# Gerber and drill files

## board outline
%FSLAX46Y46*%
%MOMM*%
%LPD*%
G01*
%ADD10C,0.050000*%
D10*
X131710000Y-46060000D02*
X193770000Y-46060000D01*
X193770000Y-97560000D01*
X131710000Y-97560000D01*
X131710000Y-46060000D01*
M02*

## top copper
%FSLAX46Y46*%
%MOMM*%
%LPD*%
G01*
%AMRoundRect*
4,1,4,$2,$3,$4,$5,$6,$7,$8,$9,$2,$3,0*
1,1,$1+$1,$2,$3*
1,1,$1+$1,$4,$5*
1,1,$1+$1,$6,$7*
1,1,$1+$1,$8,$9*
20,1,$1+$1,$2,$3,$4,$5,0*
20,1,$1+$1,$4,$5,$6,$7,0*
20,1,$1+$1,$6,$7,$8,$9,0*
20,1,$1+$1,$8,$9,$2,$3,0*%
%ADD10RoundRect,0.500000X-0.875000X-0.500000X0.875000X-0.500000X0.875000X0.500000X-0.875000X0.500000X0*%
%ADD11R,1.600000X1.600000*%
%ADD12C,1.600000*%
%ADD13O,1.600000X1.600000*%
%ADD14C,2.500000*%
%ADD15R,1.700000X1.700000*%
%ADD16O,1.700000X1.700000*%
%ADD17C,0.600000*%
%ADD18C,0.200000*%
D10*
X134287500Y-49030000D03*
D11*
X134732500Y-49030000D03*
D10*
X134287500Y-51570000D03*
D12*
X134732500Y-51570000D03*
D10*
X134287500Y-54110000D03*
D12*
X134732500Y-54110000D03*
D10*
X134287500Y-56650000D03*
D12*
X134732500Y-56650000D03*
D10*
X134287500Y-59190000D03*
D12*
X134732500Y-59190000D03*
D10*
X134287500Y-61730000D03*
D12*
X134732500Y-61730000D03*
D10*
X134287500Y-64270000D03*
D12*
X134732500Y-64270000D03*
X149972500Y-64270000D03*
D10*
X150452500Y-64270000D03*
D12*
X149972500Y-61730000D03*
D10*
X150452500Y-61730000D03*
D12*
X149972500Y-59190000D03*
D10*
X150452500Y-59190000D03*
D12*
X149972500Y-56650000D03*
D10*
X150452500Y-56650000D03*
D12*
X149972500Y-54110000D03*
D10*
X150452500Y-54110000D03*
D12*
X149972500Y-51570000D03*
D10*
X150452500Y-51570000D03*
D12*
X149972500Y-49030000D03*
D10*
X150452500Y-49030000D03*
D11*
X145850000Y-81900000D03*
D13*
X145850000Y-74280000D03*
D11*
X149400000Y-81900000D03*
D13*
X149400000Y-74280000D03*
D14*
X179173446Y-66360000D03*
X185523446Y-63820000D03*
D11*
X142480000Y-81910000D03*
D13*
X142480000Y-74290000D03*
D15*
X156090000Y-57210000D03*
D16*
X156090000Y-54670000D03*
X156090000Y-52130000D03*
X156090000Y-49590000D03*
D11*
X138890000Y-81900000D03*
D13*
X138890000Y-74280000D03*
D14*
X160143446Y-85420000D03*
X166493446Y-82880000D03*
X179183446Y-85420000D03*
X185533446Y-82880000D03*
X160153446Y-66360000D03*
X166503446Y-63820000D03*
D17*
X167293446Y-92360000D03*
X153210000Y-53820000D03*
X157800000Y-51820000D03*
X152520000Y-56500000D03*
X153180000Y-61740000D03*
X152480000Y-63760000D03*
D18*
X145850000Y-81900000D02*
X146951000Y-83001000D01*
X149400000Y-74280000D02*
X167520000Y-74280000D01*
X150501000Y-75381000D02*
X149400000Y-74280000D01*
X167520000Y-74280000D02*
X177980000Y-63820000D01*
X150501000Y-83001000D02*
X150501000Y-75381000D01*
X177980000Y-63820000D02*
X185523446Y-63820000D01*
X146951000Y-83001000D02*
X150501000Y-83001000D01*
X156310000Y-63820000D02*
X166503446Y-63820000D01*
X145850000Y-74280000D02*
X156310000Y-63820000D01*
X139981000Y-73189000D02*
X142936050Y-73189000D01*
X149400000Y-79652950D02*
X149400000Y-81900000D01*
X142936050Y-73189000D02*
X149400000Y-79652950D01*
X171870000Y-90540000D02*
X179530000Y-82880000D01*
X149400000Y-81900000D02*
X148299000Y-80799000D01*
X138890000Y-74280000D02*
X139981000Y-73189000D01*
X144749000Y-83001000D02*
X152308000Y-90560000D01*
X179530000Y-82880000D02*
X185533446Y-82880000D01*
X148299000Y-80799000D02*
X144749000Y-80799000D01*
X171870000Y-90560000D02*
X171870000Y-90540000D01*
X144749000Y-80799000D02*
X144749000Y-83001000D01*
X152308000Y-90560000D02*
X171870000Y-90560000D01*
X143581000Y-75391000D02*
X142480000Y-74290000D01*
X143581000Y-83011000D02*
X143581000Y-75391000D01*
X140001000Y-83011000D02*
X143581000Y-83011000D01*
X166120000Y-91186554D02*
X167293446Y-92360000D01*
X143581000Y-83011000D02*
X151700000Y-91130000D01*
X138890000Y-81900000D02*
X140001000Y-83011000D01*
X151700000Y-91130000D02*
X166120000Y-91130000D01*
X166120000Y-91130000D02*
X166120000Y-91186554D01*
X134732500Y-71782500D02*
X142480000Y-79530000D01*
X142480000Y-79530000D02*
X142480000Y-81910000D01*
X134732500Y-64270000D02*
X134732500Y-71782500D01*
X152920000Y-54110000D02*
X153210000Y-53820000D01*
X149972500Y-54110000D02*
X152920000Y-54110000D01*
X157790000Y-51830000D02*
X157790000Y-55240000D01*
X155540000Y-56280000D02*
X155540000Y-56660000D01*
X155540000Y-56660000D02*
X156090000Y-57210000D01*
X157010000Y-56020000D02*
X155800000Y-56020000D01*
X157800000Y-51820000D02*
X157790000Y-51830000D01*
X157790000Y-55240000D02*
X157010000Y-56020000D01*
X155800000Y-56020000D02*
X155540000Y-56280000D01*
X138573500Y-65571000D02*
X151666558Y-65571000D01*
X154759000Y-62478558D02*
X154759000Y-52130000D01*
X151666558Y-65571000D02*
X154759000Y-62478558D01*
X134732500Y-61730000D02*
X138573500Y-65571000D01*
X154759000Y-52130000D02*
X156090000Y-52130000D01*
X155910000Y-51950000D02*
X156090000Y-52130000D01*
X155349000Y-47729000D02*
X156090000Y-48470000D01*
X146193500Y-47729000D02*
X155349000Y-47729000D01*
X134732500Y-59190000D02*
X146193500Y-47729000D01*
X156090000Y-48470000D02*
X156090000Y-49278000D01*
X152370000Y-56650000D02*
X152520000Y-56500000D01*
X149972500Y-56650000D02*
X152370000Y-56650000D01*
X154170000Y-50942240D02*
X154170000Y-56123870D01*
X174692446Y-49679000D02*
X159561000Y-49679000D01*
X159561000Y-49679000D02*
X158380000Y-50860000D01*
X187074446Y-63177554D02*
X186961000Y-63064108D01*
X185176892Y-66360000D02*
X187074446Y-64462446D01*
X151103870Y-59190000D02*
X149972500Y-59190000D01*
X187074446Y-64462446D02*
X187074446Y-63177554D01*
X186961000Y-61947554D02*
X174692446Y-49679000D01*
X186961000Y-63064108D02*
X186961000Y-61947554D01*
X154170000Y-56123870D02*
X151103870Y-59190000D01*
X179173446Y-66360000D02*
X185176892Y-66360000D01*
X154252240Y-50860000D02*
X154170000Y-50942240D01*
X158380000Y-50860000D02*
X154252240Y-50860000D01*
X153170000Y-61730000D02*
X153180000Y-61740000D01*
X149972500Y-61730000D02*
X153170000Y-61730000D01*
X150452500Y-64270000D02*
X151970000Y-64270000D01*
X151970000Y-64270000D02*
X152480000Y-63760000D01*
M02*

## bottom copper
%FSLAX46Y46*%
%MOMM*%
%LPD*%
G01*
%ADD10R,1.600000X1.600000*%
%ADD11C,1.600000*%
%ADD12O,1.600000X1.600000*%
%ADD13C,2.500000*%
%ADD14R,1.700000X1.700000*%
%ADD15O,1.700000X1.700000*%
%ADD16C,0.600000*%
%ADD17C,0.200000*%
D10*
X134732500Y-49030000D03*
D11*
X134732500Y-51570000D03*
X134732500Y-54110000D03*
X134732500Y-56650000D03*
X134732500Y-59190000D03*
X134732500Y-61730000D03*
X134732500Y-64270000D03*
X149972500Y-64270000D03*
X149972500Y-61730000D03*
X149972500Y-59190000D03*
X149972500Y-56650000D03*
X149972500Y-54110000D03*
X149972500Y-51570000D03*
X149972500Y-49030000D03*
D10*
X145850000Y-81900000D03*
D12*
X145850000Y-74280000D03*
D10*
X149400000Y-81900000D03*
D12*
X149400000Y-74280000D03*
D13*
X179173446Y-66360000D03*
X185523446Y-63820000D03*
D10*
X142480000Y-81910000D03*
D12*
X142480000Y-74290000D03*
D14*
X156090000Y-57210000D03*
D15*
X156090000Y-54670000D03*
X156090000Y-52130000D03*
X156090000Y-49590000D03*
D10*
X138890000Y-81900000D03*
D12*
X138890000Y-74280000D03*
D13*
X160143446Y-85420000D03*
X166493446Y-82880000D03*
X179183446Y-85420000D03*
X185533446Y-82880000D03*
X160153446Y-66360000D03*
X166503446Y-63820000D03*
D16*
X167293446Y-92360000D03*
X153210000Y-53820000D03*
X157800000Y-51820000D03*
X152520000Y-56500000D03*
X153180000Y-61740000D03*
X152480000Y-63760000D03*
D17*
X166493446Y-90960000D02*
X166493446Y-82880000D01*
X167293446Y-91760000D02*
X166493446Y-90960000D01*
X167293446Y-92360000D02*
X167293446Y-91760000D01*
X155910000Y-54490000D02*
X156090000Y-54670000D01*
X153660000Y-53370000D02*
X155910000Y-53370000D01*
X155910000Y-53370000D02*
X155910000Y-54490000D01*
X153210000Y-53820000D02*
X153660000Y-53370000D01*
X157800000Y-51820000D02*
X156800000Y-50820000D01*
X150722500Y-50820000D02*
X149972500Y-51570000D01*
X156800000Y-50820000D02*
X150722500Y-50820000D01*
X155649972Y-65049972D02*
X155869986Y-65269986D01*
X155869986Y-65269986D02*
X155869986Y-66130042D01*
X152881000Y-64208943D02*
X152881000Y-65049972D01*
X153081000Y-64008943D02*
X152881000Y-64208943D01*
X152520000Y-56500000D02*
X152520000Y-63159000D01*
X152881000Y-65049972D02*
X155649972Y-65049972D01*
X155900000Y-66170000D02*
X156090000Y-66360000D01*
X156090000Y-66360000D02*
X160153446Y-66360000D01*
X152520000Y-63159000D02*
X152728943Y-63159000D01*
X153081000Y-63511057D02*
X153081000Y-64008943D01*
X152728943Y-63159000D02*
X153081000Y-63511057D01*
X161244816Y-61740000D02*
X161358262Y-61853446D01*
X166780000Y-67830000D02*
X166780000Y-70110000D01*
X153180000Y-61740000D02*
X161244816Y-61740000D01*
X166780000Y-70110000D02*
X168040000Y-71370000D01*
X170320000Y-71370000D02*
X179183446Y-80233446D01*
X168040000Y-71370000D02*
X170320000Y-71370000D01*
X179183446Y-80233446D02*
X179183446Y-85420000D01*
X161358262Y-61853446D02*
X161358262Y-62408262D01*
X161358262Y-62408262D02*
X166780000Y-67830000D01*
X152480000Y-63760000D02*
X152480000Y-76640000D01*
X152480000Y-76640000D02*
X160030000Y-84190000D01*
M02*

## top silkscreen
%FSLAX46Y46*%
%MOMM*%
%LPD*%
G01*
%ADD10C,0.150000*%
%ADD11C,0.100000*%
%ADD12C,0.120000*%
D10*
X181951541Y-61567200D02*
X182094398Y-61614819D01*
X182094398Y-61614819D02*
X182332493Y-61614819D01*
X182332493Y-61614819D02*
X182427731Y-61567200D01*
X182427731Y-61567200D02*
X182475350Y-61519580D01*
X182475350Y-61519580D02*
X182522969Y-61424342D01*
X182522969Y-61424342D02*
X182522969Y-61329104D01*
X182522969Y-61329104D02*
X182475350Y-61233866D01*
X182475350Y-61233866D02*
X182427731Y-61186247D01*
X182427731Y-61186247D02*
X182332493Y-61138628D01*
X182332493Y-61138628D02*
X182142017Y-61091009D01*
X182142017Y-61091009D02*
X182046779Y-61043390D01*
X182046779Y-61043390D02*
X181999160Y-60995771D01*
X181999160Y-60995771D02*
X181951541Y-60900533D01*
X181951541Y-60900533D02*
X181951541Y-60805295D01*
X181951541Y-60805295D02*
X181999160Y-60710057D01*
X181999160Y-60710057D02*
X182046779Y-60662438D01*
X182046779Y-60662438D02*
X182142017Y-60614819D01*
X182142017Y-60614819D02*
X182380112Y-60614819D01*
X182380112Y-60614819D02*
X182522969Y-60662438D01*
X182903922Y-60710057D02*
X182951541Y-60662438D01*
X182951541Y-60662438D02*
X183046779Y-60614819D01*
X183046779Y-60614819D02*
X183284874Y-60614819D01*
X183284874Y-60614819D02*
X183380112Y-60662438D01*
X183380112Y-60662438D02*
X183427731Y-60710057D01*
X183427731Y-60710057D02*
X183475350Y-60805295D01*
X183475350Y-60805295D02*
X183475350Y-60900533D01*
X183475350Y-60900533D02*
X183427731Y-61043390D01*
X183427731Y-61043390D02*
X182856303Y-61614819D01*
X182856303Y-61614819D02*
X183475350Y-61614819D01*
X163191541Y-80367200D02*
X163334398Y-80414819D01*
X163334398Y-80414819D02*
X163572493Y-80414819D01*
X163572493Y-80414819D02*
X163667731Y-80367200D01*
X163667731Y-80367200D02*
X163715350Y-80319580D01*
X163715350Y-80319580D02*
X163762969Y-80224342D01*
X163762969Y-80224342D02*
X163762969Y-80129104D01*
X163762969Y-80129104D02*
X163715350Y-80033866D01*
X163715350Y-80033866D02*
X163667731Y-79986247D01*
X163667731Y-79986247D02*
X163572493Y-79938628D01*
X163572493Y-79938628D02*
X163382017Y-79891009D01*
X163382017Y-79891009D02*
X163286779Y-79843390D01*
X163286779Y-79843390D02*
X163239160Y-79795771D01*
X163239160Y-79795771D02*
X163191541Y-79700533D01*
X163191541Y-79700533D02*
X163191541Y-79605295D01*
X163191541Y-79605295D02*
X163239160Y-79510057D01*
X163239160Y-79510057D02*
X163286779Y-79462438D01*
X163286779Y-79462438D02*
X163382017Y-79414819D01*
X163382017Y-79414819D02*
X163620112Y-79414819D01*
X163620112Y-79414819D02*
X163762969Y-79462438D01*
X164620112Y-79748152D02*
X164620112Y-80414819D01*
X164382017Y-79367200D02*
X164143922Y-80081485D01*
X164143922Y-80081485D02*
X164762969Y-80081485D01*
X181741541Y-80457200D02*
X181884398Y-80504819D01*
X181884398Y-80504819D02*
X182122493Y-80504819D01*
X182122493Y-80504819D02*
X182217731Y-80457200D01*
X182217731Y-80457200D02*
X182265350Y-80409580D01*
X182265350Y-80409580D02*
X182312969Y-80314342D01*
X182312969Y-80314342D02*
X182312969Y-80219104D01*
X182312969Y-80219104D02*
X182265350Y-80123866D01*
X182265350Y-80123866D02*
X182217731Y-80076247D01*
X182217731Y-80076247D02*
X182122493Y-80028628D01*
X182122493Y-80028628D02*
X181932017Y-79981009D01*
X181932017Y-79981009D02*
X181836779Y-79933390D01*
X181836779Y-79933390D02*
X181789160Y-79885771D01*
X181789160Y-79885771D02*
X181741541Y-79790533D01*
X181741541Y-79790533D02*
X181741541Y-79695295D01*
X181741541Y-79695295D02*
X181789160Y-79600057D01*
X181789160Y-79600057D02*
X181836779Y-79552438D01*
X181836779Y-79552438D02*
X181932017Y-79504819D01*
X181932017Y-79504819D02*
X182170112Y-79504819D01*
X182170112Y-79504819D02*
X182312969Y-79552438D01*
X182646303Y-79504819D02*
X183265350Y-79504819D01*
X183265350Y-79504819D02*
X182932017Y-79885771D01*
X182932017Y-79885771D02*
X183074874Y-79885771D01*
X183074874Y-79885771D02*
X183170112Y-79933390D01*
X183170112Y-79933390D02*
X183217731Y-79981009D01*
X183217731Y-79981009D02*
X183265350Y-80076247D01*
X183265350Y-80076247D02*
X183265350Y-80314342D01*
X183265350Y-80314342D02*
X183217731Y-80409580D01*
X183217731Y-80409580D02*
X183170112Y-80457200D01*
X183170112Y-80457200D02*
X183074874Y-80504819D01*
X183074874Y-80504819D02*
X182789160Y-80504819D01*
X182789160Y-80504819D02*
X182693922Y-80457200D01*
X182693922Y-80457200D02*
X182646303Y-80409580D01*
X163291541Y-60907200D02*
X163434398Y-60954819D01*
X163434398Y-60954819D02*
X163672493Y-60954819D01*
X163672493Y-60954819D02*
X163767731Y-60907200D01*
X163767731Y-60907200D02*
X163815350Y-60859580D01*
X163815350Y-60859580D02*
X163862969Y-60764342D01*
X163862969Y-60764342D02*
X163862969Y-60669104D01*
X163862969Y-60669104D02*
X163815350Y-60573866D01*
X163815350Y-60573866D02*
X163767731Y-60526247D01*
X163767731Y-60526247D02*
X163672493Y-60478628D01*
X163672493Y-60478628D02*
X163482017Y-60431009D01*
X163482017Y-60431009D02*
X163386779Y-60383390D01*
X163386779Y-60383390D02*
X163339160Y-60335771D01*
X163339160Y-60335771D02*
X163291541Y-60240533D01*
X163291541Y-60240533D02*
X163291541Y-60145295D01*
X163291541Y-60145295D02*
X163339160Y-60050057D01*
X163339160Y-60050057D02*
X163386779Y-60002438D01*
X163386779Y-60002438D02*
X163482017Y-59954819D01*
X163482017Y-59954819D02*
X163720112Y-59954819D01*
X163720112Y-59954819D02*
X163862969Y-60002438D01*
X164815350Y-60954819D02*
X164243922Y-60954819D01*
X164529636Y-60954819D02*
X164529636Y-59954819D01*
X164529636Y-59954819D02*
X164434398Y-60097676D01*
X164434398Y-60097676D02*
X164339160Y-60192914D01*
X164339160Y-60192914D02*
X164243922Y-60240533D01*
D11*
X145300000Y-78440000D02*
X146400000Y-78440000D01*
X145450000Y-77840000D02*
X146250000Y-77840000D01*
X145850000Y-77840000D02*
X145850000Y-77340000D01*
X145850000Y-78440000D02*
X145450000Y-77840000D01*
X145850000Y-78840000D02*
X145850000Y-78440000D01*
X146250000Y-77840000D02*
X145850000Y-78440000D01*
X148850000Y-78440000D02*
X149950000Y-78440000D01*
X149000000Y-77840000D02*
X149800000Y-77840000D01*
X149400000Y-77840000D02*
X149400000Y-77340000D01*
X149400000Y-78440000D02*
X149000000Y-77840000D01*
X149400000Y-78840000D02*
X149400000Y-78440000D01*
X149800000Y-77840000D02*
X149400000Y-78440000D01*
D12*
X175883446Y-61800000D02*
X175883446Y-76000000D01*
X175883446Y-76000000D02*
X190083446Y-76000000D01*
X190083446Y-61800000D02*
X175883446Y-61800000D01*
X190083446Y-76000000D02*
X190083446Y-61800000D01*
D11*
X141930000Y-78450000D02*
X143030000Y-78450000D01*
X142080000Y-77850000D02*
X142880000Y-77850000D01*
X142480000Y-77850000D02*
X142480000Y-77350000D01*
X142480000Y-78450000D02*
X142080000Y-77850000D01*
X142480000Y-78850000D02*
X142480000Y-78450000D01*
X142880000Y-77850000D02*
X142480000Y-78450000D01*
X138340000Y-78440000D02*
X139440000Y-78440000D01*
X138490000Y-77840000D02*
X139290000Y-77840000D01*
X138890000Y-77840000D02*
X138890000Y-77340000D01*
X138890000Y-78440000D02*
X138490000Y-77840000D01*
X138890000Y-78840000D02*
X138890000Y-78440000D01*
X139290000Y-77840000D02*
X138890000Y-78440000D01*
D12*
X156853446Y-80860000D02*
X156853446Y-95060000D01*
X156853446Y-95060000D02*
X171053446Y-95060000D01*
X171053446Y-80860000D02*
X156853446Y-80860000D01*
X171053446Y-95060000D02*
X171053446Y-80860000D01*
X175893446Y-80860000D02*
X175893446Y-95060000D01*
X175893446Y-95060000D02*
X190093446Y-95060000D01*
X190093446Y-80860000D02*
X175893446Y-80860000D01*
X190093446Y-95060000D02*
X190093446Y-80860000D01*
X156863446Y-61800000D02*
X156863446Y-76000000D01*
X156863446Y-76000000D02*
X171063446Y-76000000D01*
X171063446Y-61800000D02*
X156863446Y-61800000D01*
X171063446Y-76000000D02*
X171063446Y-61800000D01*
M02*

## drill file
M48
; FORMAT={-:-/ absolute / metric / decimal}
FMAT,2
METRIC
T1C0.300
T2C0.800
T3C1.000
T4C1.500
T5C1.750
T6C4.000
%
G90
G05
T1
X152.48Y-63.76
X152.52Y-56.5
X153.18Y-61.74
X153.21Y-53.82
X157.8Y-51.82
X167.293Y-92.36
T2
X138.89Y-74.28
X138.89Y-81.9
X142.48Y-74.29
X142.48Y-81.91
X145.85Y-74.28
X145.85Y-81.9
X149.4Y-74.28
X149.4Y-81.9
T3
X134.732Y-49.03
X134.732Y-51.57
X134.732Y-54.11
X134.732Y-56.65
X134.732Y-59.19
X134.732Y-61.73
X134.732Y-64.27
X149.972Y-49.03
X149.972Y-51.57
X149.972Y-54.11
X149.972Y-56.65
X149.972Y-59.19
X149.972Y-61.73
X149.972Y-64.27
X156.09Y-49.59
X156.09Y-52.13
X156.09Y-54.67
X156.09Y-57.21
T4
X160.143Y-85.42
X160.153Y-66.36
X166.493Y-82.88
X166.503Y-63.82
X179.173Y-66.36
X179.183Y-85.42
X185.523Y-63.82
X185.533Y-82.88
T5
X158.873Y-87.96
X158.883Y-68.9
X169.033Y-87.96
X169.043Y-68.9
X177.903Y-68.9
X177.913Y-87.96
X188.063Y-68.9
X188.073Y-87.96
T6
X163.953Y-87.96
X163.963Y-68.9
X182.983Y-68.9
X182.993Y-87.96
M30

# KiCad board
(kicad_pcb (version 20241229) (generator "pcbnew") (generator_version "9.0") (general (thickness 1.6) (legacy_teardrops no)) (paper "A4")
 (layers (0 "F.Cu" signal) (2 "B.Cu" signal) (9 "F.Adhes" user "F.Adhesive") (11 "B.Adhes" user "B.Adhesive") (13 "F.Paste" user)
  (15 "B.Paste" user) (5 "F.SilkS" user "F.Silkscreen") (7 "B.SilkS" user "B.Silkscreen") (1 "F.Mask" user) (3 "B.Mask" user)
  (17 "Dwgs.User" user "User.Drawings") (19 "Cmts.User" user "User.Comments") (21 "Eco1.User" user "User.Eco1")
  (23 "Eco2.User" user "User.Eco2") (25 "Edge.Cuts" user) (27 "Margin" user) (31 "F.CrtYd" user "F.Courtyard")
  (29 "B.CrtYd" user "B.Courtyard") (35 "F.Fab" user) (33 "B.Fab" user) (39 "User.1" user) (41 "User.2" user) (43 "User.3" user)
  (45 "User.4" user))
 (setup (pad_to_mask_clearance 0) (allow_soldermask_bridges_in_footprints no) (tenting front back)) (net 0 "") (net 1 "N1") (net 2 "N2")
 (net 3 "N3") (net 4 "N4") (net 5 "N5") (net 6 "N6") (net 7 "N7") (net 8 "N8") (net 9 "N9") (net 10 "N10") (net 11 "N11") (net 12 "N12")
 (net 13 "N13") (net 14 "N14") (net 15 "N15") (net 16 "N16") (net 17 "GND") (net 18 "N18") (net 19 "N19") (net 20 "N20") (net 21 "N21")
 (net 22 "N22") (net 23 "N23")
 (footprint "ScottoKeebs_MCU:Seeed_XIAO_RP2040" (layer "F.Cu") (at 142.3525 56.65)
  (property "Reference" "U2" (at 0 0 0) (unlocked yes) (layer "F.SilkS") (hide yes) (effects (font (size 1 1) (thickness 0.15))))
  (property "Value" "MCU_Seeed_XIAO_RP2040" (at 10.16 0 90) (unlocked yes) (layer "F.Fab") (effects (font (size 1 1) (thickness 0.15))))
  (pad "1" smd roundrect (at -8.065 -7.62) (size 2.75 2) (layers "F.Cu" "F.Mask" "F.Paste") (roundrect_rratio 0.25) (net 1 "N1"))
  (pad "1" thru_hole rect (at -7.62 -7.62 90) (size 1.6 1.6) (drill 1) (layers "*.Cu" "*.Mask") (remove_unused_layers no) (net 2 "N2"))
  (pad "2" smd roundrect (at -8.065 -5.08) (size 2.75 2) (layers "F.Cu" "F.Mask" "F.Paste") (roundrect_rratio 0.25) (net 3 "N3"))
  (pad "2" thru_hole circle (at -7.62 -5.08 90) (size 1.6 1.6) (drill 1) (layers "*.Cu" "*.Mask") (remove_unused_layers no) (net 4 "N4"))
  (pad "3" smd roundrect (at -8.065 -2.54) (size 2.75 2) (layers "F.Cu" "F.Mask" "F.Paste") (roundrect_rratio 0.25) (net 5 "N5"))
  (pad "3" thru_hole circle (at -7.62 -2.54 90) (size 1.6 1.6) (drill 1) (layers "*.Cu" "*.Mask") (remove_unused_layers no) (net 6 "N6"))
  (pad "4" smd roundrect (at -8.065 0) (size 2.75 2) (layers "F.Cu" "F.Mask" "F.Paste") (roundrect_rratio 0.25) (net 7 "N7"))
  (pad "4" thru_hole circle (at -7.62 0 90) (size 1.6 1.6) (drill 1) (layers "*.Cu" "*.Mask") (remove_unused_layers no) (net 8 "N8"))
  (pad "5" smd roundrect (at -8.065 2.54) (size 2.75 2) (layers "F.Cu" "F.Mask" "F.Paste") (roundrect_rratio 0.25) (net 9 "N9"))
  (pad "5" thru_hole circle (at -7.62 2.54 90) (size 1.6 1.6) (drill 1) (layers "*.Cu" "*.Mask") (remove_unused_layers no) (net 9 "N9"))
  (pad "6" smd roundrect (at -8.065 5.08) (size 2.75 2) (layers "F.Cu" "F.Mask" "F.Paste") (roundrect_rratio 0.25) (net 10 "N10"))
  (pad "6" thru_hole circle (at -7.62 5.08 90) (size 1.6 1.6) (drill 1) (layers "*.Cu" "*.Mask") (remove_unused_layers no) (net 10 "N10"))
  (pad "7" smd roundrect (at -8.065 7.62) (size 2.75 2) (layers "F.Cu" "F.Mask" "F.Paste") (roundrect_rratio 0.25) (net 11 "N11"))
  (pad "7" thru_hole circle (at -7.62 7.62 90) (size 1.6 1.6) (drill 1) (layers "*.Cu" "*.Mask") (remove_unused_layers no) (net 11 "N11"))
  (pad "8" thru_hole circle (at 7.62 7.62 90) (size 1.6 1.6) (drill 1) (layers "*.Cu" "*.Mask") (remove_unused_layers no) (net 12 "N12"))
  (pad "8" smd roundrect (at 8.1 7.62) (size 2.75 2) (layers "F.Cu" "F.Mask" "F.Paste") (roundrect_rratio 0.25) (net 12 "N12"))
  (pad "9" thru_hole circle (at 7.62 5.08 90) (size 1.6 1.6) (drill 1) (layers "*.Cu" "*.Mask") (remove_unused_layers no) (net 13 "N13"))
  (pad "9" smd roundrect (at 8.1 5.08) (size 2.75 2) (layers "F.Cu" "F.Mask" "F.Paste") (roundrect_rratio 0.25) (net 13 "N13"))
  (pad "10" thru_hole circle (at 7.62 2.54 90) (size 1.6 1.6) (drill 1) (layers "*.Cu" "*.Mask") (remove_unused_layers no) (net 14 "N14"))
  (pad "10" smd roundrect (at 8.1 2.54) (size 2.75 2) (layers "F.Cu" "F.Mask" "F.Paste") (roundrect_rratio 0.25) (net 14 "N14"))
  (pad "11" thru_hole circle (at 7.62 0 90) (size 1.6 1.6) (drill 1) (layers "*.Cu" "*.Mask") (remove_unused_layers no) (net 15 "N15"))
  (pad "11" smd roundrect (at 8.1 0) (size 2.75 2) (layers "F.Cu" "F.Mask" "F.Paste") (roundrect_rratio 0.25) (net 15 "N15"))
  (pad "12" thru_hole circle (at 7.62 -2.54 90) (size 1.6 1.6) (drill 1) (layers "*.Cu" "*.Mask") (remove_unused_layers no) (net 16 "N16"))
  (pad "12" smd roundrect (at 8.1 -2.54) (size 2.75 2) (layers "F.Cu" "F.Mask" "F.Paste") (roundrect_rratio 0.25) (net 16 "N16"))
  (pad "13" thru_hole circle (at 7.62 -5.08 90) (size 1.6 1.6) (drill 1) (layers "*.Cu" "*.Mask") (remove_unused_layers no) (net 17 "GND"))
  (pad "13" smd roundrect (at 8.1 -5.08) (size 2.75 2) (layers "F.Cu" "F.Mask" "F.Paste") (roundrect_rratio 0.25) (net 17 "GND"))
  (pad "14" thru_hole circle (at 7.62 -7.62 90) (size 1.6 1.6) (drill 1) (layers "*.Cu" "*.Mask") (remove_unused_layers no) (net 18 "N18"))
  (pad "14" smd roundrect (at 8.1 -7.62) (size 2.75 2) (layers "F.Cu" "F.Mask" "F.Paste") (roundrect_rratio 0.25) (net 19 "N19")))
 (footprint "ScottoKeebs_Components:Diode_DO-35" (layer "F.Cu") (at 145.85 81.9 90)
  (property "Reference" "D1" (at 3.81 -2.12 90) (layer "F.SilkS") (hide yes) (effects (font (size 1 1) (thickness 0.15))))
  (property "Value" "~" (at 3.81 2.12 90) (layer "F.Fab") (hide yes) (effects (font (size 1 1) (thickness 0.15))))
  (fp_line (start 3.46 -0.55) (end 3.46 0.55) (stroke (width 0.1) (type solid)) (layer "F.SilkS"))
  (fp_line (start 4.06 -0.4) (end 4.06 0.4) (stroke (width 0.1) (type solid)) (layer "F.SilkS"))
  (fp_line (start 4.06 0) (end 4.56 0) (stroke (width 0.1) (type solid)) (layer "F.SilkS"))
  (fp_line (start 3.46 0) (end 4.06 -0.4) (stroke (width 0.1) (type solid)) (layer "F.SilkS"))
  (fp_line (start 3.06 0) (end 3.46 0) (stroke (width 0.1) (type solid)) (layer "F.SilkS"))
  (fp_line (start 4.06 0.4) (end 3.46 0) (stroke (width 0.1) (type solid)) (layer "F.SilkS"))
  (pad "1" thru_hole rect (at 0 0 90) (size 1.6 1.6) (drill 0.8) (layers "*.Cu" "*.Mask") (remove_unused_layers no) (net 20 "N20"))
  (pad "2" thru_hole oval (at 7.62 0 90) (size 1.6 1.6) (drill 0.8) (layers "*.Cu" "*.Mask") (remove_unused_layers no) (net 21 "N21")))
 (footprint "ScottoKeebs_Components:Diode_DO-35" (layer "F.Cu") (at 149.4 81.9 90)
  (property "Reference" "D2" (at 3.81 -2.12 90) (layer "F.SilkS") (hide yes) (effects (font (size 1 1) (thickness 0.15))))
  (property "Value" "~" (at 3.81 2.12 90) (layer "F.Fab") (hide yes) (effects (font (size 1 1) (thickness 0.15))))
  (fp_line (start 3.46 -0.55) (end 3.46 0.55) (stroke (width 0.1) (type solid)) (layer "F.SilkS"))
  (fp_line (start 4.06 -0.4) (end 4.06 0.4) (stroke (width 0.1) (type solid)) (layer "F.SilkS"))
  (fp_line (start 4.06 0) (end 4.56 0) (stroke (width 0.1) (type solid)) (layer "F.SilkS"))
  (fp_line (start 3.46 0) (end 4.06 -0.4) (stroke (width 0.1) (type solid)) (layer "F.SilkS"))
  (fp_line (start 3.06 0) (end 3.46 0) (stroke (width 0.1) (type solid)) (layer "F.SilkS"))
  (fp_line (start 4.06 0.4) (end 3.46 0) (stroke (width 0.1) (type solid)) (layer "F.SilkS"))
  (pad "1" thru_hole rect (at 0 0 90) (size 1.6 1.6) (drill 0.8) (layers "*.Cu" "*.Mask") (remove_unused_layers no) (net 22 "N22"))
  (pad "2" thru_hole oval (at 7.62 0 90) (size 1.6 1.6) (drill 0.8) (layers "*.Cu" "*.Mask") (remove_unused_layers no) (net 20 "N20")))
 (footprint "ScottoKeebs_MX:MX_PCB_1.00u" (layer "F.Cu") (at 182.983446 68.9)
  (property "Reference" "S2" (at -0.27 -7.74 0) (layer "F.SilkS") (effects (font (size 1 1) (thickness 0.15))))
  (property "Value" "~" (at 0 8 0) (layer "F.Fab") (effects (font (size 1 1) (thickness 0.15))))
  (fp_line (start -7.1 -7.1) (end -7.1 7.1) (stroke (width 0.12) (type solid)) (layer "F.SilkS"))
  (fp_line (start -7.1 7.1) (end 7.1 7.1) (stroke (width 0.12) (type solid)) (layer "F.SilkS"))
  (fp_line (start 7.1 -7.1) (end -7.1 -7.1) (stroke (width 0.12) (type solid)) (layer "F.SilkS"))
  (fp_line (start 7.1 7.1) (end 7.1 -7.1) (stroke (width 0.12) (type solid)) (layer "F.SilkS"))
  (pad "" np_thru_hole circle (at -5.08 0) (size 1.75 1.75) (drill 1.75) (layers "*.Cu" "*.Mask"))
  (pad "" np_thru_hole circle (at 0 0) (size 4 4) (drill 4) (layers "*.Cu" "*.Mask"))
  (pad "" np_thru_hole circle (at 5.08 0) (size 1.75 1.75) (drill 1.75) (layers "*.Cu" "*.Mask"))
  (pad "1" thru_hole circle (at -3.81 -2.54) (size 2.5 2.5) (drill 1.5) (layers "*.Cu" "*.Mask") (remove_unused_layers no) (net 14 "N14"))
  (pad "2" thru_hole circle (at 2.54 -5.08) (size 2.5 2.5) (drill 1.5) (layers "*.Cu" "*.Mask") (remove_unused_layers no) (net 20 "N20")))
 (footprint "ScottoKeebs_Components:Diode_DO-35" (layer "F.Cu") (at 142.48 81.91 90)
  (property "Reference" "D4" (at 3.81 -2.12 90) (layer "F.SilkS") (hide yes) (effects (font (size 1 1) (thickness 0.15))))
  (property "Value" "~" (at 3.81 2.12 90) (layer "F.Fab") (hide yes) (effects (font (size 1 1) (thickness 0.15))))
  (fp_line (start 3.46 -0.55) (end 3.46 0.55) (stroke (width 0.1) (type solid)) (layer "F.SilkS"))
  (fp_line (start 4.06 -0.4) (end 4.06 0.4) (stroke (width 0.1) (type solid)) (layer "F.SilkS"))
  (fp_line (start 4.06 0) (end 4.56 0) (stroke (width 0.1) (type solid)) (layer "F.SilkS"))
  (fp_line (start 3.46 0) (end 4.06 -0.4) (stroke (width 0.1) (type solid)) (layer "F.SilkS"))
  (fp_line (start 3.06 0) (end 3.46 0) (stroke (width 0.1) (type solid)) (layer "F.SilkS"))
  (fp_line (start 4.06 0.4) (end 3.46 0) (stroke (width 0.1) (type solid)) (layer "F.SilkS"))
  (pad "1" thru_hole rect (at 0 0 90) (size 1.6 1.6) (drill 0.8) (layers "*.Cu" "*.Mask") (remove_unused_layers no) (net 11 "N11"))
  (pad "2" thru_hole oval (at 7.62 0 90) (size 1.6 1.6) (drill 0.8) (layers "*.Cu" "*.Mask") (remove_unused_layers no) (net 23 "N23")))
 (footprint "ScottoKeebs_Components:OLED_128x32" (layer "F.Cu") (at 154.49 47.41)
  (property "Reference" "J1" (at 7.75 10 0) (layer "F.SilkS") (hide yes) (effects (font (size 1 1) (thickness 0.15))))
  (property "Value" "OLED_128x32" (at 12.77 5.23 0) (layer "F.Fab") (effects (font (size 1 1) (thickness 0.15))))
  (pad "1" thru_hole rect (at 1.6 9.8 180) (size 1.7 1.7) (drill 1) (layers "*.Cu" "*.Mask") (remove_unused_layers no) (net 17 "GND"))
  (pad "2" thru_hole oval (at 1.6 7.26 180) (size 1.7 1.7) (drill 1) (layers "*.Cu" "*.Mask") (remove_unused_layers no) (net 16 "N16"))
  (pad "3" thru_hole oval (at 1.6 4.72 180) (size 1.7 1.7) (drill 1) (layers "*.Cu" "*.Mask") (remove_unused_layers no) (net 10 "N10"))
  (pad "4" thru_hole oval (at 1.6 2.18 180) (size 1.7 1.7) (drill 1) (layers "*.Cu" "*.Mask") (remove_unused_layers no) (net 9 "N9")))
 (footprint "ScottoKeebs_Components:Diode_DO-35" (layer "F.Cu") (at 138.89 81.9 90)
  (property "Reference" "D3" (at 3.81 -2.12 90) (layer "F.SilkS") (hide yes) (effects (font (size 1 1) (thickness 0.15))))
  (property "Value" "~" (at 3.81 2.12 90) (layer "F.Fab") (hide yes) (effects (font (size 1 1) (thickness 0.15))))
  (fp_line (start 3.46 -0.55) (end 3.46 0.55) (stroke (width 0.1) (type solid)) (layer "F.SilkS"))
  (fp_line (start 4.06 -0.4) (end 4.06 0.4) (stroke (width 0.1) (type solid)) (layer "F.SilkS"))
  (fp_line (start 4.06 0) (end 4.56 0) (stroke (width 0.1) (type solid)) (layer "F.SilkS"))
  (fp_line (start 3.46 0) (end 4.06 -0.4) (stroke (width 0.1) (type solid)) (layer "F.SilkS"))
  (fp_line (start 3.06 0) (end 3.46 0) (stroke (width 0.1) (type solid)) (layer "F.SilkS"))
  (fp_line (start 4.06 0.4) (end 3.46 0) (stroke (width 0.1) (type solid)) (layer "F.SilkS"))
  (pad "1" thru_hole rect (at 0 0 90) (size 1.6 1.6) (drill 0.8) (layers "*.Cu" "*.Mask") (remove_unused_layers no) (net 23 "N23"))
  (pad "2" thru_hole oval (at 7.62 0 90) (size 1.6 1.6) (drill 0.8) (layers "*.Cu" "*.Mask") (remove_unused_layers no) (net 22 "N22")))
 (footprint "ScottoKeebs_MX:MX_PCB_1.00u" (layer "F.Cu") (at 163.953446 87.96)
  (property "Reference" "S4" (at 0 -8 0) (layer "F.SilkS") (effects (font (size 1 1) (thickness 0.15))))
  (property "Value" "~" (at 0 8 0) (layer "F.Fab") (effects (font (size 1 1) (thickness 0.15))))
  (fp_line (start -7.1 -7.1) (end -7.1 7.1) (stroke (width 0.12) (type solid)) (layer "F.SilkS"))
  (fp_line (start -7.1 7.1) (end 7.1 7.1) (stroke (width 0.12) (type solid)) (layer "F.SilkS"))
  (fp_line (start 7.1 -7.1) (end -7.1 -7.1) (stroke (width 0.12) (type solid)) (layer "F.SilkS"))
  (fp_line (start 7.1 7.1) (end 7.1 -7.1) (stroke (width 0.12) (type solid)) (layer "F.SilkS"))
  (pad "" np_thru_hole circle (at -5.08 0) (size 1.75 1.75) (drill 1.75) (layers "*.Cu" "*.Mask"))
  (pad "" np_thru_hole circle (at 0 0) (size 4 4) (drill 4) (layers "*.Cu" "*.Mask"))
  (pad "" np_thru_hole circle (at 5.08 0) (size 1.75 1.75) (drill 1.75) (layers "*.Cu" "*.Mask"))
  (pad "1" thru_hole circle (at -3.81 -2.54) (size 2.5 2.5) (drill 1.5) (layers "*.Cu" "*.Mask") (remove_unused_layers no) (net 12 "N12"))
  (pad "2" thru_hole circle (at 2.54 -5.08) (size 2.5 2.5) (drill 1.5) (layers "*.Cu" "*.Mask") (remove_unused_layers no) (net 23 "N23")))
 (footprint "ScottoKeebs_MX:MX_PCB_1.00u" (layer "F.Cu") (at 182.993446 87.96)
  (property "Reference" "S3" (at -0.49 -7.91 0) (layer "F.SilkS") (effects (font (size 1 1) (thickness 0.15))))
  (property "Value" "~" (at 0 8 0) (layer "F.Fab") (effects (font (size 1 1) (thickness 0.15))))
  (fp_line (start -7.1 -7.1) (end -7.1 7.1) (stroke (width 0.12) (type solid)) (layer "F.SilkS"))
  (fp_line (start -7.1 7.1) (end 7.1 7.1) (stroke (width 0.12) (type solid)) (layer "F.SilkS"))
  (fp_line (start 7.1 -7.1) (end -7.1 -7.1) (stroke (width 0.12) (type solid)) (layer "F.SilkS"))
  (fp_line (start 7.1 7.1) (end 7.1 -7.1) (stroke (width 0.12) (type solid)) (layer "F.SilkS"))
  (pad "" np_thru_hole circle (at -5.08 0) (size 1.75 1.75) (drill 1.75) (layers "*.Cu" "*.Mask"))
  (pad "" np_thru_hole circle (at 0 0) (size 4 4) (drill 4) (layers "*.Cu" "*.Mask"))
  (pad "" np_thru_hole circle (at 5.08 0) (size 1.75 1.75) (drill 1.75) (layers "*.Cu" "*.Mask"))
  (pad "1" thru_hole circle (at -3.81 -2.54) (size 2.5 2.5) (drill 1.5) (layers "*.Cu" "*.Mask") (remove_unused_layers no) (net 13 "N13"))
  (pad "2" thru_hole circle (at 2.54 -5.08) (size 2.5 2.5) (drill 1.5) (layers "*.Cu" "*.Mask") (remove_unused_layers no) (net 22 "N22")))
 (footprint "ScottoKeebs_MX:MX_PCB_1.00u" (layer "F.Cu") (at 163.963446 68.9)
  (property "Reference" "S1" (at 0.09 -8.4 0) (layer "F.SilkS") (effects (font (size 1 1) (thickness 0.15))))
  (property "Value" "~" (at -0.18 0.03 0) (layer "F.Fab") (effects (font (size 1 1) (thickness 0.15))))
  (fp_line (start -7.1 -7.1) (end -7.1 7.1) (stroke (width 0.12) (type solid)) (layer "F.SilkS"))
  (fp_line (start -7.1 7.1) (end 7.1 7.1) (stroke (width 0.12) (type solid)) (layer "F.SilkS"))
  (fp_line (start 7.1 -7.1) (end -7.1 -7.1) (stroke (width 0.12) (type solid)) (layer "F.SilkS"))
  (fp_line (start 7.1 7.1) (end 7.1 -7.1) (stroke (width 0.12) (type solid)) (layer "F.SilkS"))
  (pad "" np_thru_hole circle (at -5.08 0) (size 1.75 1.75) (drill 1.75) (layers "*.Cu" "*.Mask"))
  (pad "" np_thru_hole circle (at 0 0) (size 4 4) (drill 4) (layers "*.Cu" "*.Mask"))
  (pad "" np_thru_hole circle (at 5.08 0) (size 1.75 1.75) (drill 1.75) (layers "*.Cu" "*.Mask"))
  (pad "1" thru_hole circle (at -3.81 -2.54) (size 2.5 2.5) (drill 1.5) (layers "*.Cu" "*.Mask") (remove_unused_layers no) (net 15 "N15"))
  (pad "2" thru_hole circle (at 2.54 -5.08) (size 2.5 2.5) (drill 1.5) (layers "*.Cu" "*.Mask") (remove_unused_layers no) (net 21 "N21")))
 (gr_rect (start 131.71 46.06) (end 193.77 97.56) (stroke (width 0.05) (type default)) (fill no) (layer "Edge.Cuts"))
 (segment (start 145.85 81.9) (end 146.951 83.001) (width 0.2) (layer "F.Cu") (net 20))
 (segment (start 149.4 74.28) (end 167.52 74.28) (width 0.2) (layer "F.Cu") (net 20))
 (segment (start 150.501 75.381) (end 149.4 74.28) (width 0.2) (layer "F.Cu") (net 20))
 (segment (start 167.52 74.28) (end 177.98 63.82) (width 0.2) (layer "F.Cu") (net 20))
 (segment (start 150.501 83.001) (end 150.501 75.381) (width 0.2) (layer "F.Cu") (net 20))
 (segment (start 177.98 63.82) (end 185.523446 63.82) (width 0.2) (layer "F.Cu") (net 20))
 (segment (start 146.951 83.001) (end 150.501 83.001) (width 0.2) (layer "F.Cu") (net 20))
 (segment (start 156.31 63.82) (end 166.503446 63.82) (width 0.2) (layer "F.Cu") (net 21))
 (segment (start 145.85 74.28) (end 156.31 63.82) (width 0.2) (layer "F.Cu") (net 21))
 (segment (start 139.981 73.189) (end 142.93605 73.189) (width 0.2) (layer "F.Cu") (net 22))
 (segment (start 149.4 79.65295) (end 149.4 81.9) (width 0.2) (layer "F.Cu") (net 22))
 (segment (start 142.93605 73.189) (end 149.4 79.65295) (width 0.2) (layer "F.Cu") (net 22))
 (segment (start 171.87 90.54) (end 179.53 82.88) (width 0.2) (layer "F.Cu") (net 22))
 (segment (start 149.4 81.9) (end 148.299 80.799) (width 0.2) (layer "F.Cu") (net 22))
 (segment (start 138.89 74.28) (end 139.981 73.189) (width 0.2) (layer "F.Cu") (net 22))
 (segment (start 144.749 83.001) (end 152.308 90.56) (width 0.2) (layer "F.Cu") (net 22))
 (segment (start 179.53 82.88) (end 185.533446 82.88) (width 0.2) (layer "F.Cu") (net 22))
 (segment (start 148.299 80.799) (end 144.749 80.799) (width 0.2) (layer "F.Cu") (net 22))
 (segment (start 171.87 90.56) (end 171.87 90.54) (width 0.2) (layer "F.Cu") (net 22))
 (segment (start 144.749 80.799) (end 144.749 83.001) (width 0.2) (layer "F.Cu") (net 22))
 (segment (start 152.308 90.56) (end 171.87 90.56) (width 0.2) (layer "F.Cu") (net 22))
 (segment (start 143.581 75.391) (end 142.48 74.29) (width 0.2) (layer "F.Cu") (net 23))
 (segment (start 143.581 83.011) (end 143.581 75.391) (width 0.2) (layer "F.Cu") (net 23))
 (segment (start 140.001 83.011) (end 143.581 83.011) (width 0.2) (layer "F.Cu") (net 23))
 (segment (start 166.12 91.186554) (end 167.293446 92.36) (width 0.2) (layer "F.Cu") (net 23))
 (segment (start 143.581 83.011) (end 151.7 91.13) (width 0.2) (layer "F.Cu") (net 23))
 (segment (start 138.89 81.9) (end 140.001 83.011) (width 0.2) (layer "F.Cu") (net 23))
 (segment (start 151.7 91.13) (end 166.12 91.13) (width 0.2) (layer "F.Cu") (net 23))
 (segment (start 166.12 91.13) (end 166.12 91.186554) (width 0.2) (layer "F.Cu") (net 23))
 (via (at 167.293446 92.36) (size 0.6) (drill 0.3) (layers "F.Cu" "B.Cu") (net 23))
 (segment (start 166.493446 90.96) (end 166.493446 82.88) (width 0.2) (layer "B.Cu") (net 23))
 (segment (start 167.293446 91.76) (end 166.493446 90.96) (width 0.2) (layer "B.Cu") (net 23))
 (segment (start 167.293446 92.36) (end 167.293446 91.76) (width 0.2) (layer "B.Cu") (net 23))
 (segment (start 134.7325 71.7825) (end 142.48 79.53) (width 0.2) (layer "F.Cu") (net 11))
 (segment (start 142.48 79.53) (end 142.48 81.91) (width 0.2) (layer "F.Cu") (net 11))
 (segment (start 134.7325 64.27) (end 134.7325 71.7825) (width 0.2) (layer "F.Cu") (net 11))
 (segment (start 152.92 54.11) (end 153.21 53.82) (width 0.2) (layer "F.Cu") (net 16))
 (segment (start 149.9725 54.11) (end 152.92 54.11) (width 0.2) (layer "F.Cu") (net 16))
 (via (at 153.21 53.82) (size 0.6) (drill 0.3) (layers "F.Cu" "B.Cu") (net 16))
 (segment (start 155.91 54.49) (end 156.09 54.67) (width 0.2) (layer "B.Cu") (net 16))
 (segment (start 153.66 53.37) (end 155.91 53.37) (width 0.2) (layer "B.Cu") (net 16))
 (segment (start 155.91 53.37) (end 155.91 54.49) (width 0.2) (layer "B.Cu") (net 16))
 (segment (start 153.21 53.82) (end 153.66 53.37) (width 0.2) (layer "B.Cu") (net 16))
 (segment (start 157.79 51.83) (end 157.79 55.24) (width 0.2) (layer "F.Cu") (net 17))
 (segment (start 155.54 56.28) (end 155.54 56.66) (width 0.2) (layer "F.Cu") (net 17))
 (segment (start 155.54 56.66) (end 156.09 57.21) (width 0.2) (layer "F.Cu") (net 17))
 (segment (start 157.01 56.02) (end 155.8 56.02) (width 0.2) (layer "F.Cu") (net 17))
 (segment (start 157.8 51.82) (end 157.79 51.83) (width 0.2) (layer "F.Cu") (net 17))
 (segment (start 157.79 55.24) (end 157.01 56.02) (width 0.2) (layer "F.Cu") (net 17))
 (segment (start 155.8 56.02) (end 155.54 56.28) (width 0.2) (layer "F.Cu") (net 17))
 (via (at 157.8 51.82) (size 0.6) (drill 0.3) (layers "F.Cu" "B.Cu") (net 17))
 (segment (start 157.8 51.82) (end 156.8 50.82) (width 0.2) (layer "B.Cu") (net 17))
 (segment (start 150.7225 50.82) (end 149.9725 51.57) (width 0.2) (layer "B.Cu") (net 17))
 (segment (start 156.8 50.82) (end 150.7225 50.82) (width 0.2) (layer "B.Cu") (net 17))
 (segment (start 138.5735 65.571) (end 151.666558 65.571) (width 0.2) (layer "F.Cu") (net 10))
 (segment (start 154.759 62.478558) (end 154.759 52.13) (width 0.2) (layer "F.Cu") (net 10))
 (segment (start 151.666558 65.571) (end 154.759 62.478558) (width 0.2) (layer "F.Cu") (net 10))
 (segment (start 134.7325 61.73) (end 138.5735 65.571) (width 0.2) (layer "F.Cu") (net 10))
 (segment (start 154.759 52.13) (end 156.09 52.13) (width 0.2) (layer "F.Cu") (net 10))
 (segment (start 155.91 51.95) (end 156.09 52.13) (width 0.2) (layer "F.Cu") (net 10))
 (segment (start 155.349 47.729) (end 156.09 48.47) (width 0.2) (layer "F.Cu") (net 9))
 (segment (start 146.1935 47.729) (end 155.349 47.729) (width 0.2) (layer "F.Cu") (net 9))
 (segment (start 134.7325 59.19) (end 146.1935 47.729) (width 0.2) (layer "F.Cu") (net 9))
 (segment (start 156.09 48.47) (end 156.09 49.278) (width 0.2) (layer "F.Cu") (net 9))
 (segment (start 152.37 56.65) (end 152.52 56.5) (width 0.2) (layer "F.Cu") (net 15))
 (segment (start 149.9725 56.65) (end 152.37 56.65) (width 0.2) (layer "F.Cu") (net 15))
 (via (at 152.52 56.5) (size 0.6) (drill 0.3) (layers "F.Cu" "B.Cu") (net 15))
 (segment (start 155.649972 65.049972) (end 155.869986 65.269986) (width 0.2) (layer "B.Cu") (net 15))
 (segment (start 155.869986 65.269986) (end 155.869986 66.130042) (width 0.2) (layer "B.Cu") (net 15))
 (segment (start 152.881 64.208943) (end 152.881 65.049972) (width 0.2) (layer "B.Cu") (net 15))
 (segment (start 153.081 64.008943) (end 152.881 64.208943) (width 0.2) (layer "B.Cu") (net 15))
 (segment (start 152.52 56.5) (end 152.52 63.159) (width 0.2) (layer "B.Cu") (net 15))
 (segment (start 152.881 65.049972) (end 155.649972 65.049972) (width 0.2) (layer "B.Cu") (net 15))
 (segment (start 155.9 66.17) (end 156.09 66.36) (width 0.2) (layer "B.Cu") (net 15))
 (segment (start 156.09 66.36) (end 160.153446 66.36) (width 0.2) (layer "B.Cu") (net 15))
 (segment (start 152.52 63.159) (end 152.728943 63.159) (width 0.2) (layer "B.Cu") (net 15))
 (segment (start 153.081 63.511057) (end 153.081 64.008943) (width 0.2) (layer "B.Cu") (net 15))
 (segment (start 152.728943 63.159) (end 153.081 63.511057) (width 0.2) (layer "B.Cu") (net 15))
 (segment (start 154.17 50.94224) (end 154.17 56.12387) (width 0.2) (layer "F.Cu") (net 14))
 (segment (start 174.692446 49.679) (end 159.561 49.679) (width 0.2) (layer "F.Cu") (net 14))
 (segment (start 159.561 49.679) (end 158.38 50.86) (width 0.2) (layer "F.Cu") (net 14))
 (segment (start 187.074446 63.177554) (end 186.961 63.064108) (width 0.2) (layer "F.Cu") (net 14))
 (segment (start 185.176892 66.36) (end 187.074446 64.462446) (width 0.2) (layer "F.Cu") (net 14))
 (segment (start 151.10387 59.19) (end 149.9725 59.19) (width 0.2) (layer "F.Cu") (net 14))
 (segment (start 187.074446 64.462446) (end 187.074446 63.177554) (width 0.2) (layer "F.Cu") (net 14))
 (segment (start 186.961 61.947554) (end 174.692446 49.679) (width 0.2) (layer "F.Cu") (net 14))
 (segment (start 186.961 63.064108) (end 186.961 61.947554) (width 0.2) (layer "F.Cu") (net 14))
 (segment (start 154.17 56.12387) (end 151.10387 59.19) (width 0.2) (layer "F.Cu") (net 14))
 (segment (start 179.173446 66.36) (end 185.176892 66.36) (width 0.2) (layer "F.Cu") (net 14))
 (segment (start 154.25224 50.86) (end 154.17 50.94224) (width 0.2) (layer "F.Cu") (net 14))
 (segment (start 158.38 50.86) (end 154.25224 50.86) (width 0.2) (layer "F.Cu") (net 14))
 (segment (start 153.17 61.73) (end 153.18 61.74) (width 0.2) (layer "F.Cu") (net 13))
 (segment (start 149.9725 61.73) (end 153.17 61.73) (width 0.2) (layer "F.Cu") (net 13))
 (via (at 153.18 61.74) (size 0.6) (drill 0.3) (layers "F.Cu" "B.Cu") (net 13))
 (segment (start 161.244816 61.74) (end 161.358262 61.853446) (width 0.2) (layer "B.Cu") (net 13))
 (segment (start 166.78 67.83) (end 166.78 70.11) (width 0.2) (layer "B.Cu") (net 13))
 (segment (start 153.18 61.74) (end 161.244816 61.74) (width 0.2) (layer "B.Cu") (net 13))
 (segment (start 166.78 70.11) (end 168.04 71.37) (width 0.2) (layer "B.Cu") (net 13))
 (segment (start 170.32 71.37) (end 179.183446 80.233446) (width 0.2) (layer "B.Cu") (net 13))
 (segment (start 168.04 71.37) (end 170.32 71.37) (width 0.2) (layer "B.Cu") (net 13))
 (segment (start 179.183446 80.233446) (end 179.183446 85.42) (width 0.2) (layer "B.Cu") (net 13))
 (segment (start 161.358262 61.853446) (end 161.358262 62.408262) (width 0.2) (layer "B.Cu") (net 13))
 (segment (start 161.358262 62.408262) (end 166.78 67.83) (width 0.2) (layer "B.Cu") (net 13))
 (segment (start 150.4525 64.27) (end 151.97 64.27) (width 0.2) (layer "F.Cu") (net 12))
 (segment (start 151.97 64.27) (end 152.48 63.76) (width 0.2) (layer "F.Cu") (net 12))
 (via (at 152.48 63.76) (size 0.6) (drill 0.3) (layers "F.Cu" "B.Cu") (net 12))
 (segment (start 152.48 63.76) (end 152.48 76.64) (width 0.2) (layer "B.Cu") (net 12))
 (segment (start 152.48 76.64) (end 160.03 84.19) (width 0.2) (layer "B.Cu") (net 12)))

